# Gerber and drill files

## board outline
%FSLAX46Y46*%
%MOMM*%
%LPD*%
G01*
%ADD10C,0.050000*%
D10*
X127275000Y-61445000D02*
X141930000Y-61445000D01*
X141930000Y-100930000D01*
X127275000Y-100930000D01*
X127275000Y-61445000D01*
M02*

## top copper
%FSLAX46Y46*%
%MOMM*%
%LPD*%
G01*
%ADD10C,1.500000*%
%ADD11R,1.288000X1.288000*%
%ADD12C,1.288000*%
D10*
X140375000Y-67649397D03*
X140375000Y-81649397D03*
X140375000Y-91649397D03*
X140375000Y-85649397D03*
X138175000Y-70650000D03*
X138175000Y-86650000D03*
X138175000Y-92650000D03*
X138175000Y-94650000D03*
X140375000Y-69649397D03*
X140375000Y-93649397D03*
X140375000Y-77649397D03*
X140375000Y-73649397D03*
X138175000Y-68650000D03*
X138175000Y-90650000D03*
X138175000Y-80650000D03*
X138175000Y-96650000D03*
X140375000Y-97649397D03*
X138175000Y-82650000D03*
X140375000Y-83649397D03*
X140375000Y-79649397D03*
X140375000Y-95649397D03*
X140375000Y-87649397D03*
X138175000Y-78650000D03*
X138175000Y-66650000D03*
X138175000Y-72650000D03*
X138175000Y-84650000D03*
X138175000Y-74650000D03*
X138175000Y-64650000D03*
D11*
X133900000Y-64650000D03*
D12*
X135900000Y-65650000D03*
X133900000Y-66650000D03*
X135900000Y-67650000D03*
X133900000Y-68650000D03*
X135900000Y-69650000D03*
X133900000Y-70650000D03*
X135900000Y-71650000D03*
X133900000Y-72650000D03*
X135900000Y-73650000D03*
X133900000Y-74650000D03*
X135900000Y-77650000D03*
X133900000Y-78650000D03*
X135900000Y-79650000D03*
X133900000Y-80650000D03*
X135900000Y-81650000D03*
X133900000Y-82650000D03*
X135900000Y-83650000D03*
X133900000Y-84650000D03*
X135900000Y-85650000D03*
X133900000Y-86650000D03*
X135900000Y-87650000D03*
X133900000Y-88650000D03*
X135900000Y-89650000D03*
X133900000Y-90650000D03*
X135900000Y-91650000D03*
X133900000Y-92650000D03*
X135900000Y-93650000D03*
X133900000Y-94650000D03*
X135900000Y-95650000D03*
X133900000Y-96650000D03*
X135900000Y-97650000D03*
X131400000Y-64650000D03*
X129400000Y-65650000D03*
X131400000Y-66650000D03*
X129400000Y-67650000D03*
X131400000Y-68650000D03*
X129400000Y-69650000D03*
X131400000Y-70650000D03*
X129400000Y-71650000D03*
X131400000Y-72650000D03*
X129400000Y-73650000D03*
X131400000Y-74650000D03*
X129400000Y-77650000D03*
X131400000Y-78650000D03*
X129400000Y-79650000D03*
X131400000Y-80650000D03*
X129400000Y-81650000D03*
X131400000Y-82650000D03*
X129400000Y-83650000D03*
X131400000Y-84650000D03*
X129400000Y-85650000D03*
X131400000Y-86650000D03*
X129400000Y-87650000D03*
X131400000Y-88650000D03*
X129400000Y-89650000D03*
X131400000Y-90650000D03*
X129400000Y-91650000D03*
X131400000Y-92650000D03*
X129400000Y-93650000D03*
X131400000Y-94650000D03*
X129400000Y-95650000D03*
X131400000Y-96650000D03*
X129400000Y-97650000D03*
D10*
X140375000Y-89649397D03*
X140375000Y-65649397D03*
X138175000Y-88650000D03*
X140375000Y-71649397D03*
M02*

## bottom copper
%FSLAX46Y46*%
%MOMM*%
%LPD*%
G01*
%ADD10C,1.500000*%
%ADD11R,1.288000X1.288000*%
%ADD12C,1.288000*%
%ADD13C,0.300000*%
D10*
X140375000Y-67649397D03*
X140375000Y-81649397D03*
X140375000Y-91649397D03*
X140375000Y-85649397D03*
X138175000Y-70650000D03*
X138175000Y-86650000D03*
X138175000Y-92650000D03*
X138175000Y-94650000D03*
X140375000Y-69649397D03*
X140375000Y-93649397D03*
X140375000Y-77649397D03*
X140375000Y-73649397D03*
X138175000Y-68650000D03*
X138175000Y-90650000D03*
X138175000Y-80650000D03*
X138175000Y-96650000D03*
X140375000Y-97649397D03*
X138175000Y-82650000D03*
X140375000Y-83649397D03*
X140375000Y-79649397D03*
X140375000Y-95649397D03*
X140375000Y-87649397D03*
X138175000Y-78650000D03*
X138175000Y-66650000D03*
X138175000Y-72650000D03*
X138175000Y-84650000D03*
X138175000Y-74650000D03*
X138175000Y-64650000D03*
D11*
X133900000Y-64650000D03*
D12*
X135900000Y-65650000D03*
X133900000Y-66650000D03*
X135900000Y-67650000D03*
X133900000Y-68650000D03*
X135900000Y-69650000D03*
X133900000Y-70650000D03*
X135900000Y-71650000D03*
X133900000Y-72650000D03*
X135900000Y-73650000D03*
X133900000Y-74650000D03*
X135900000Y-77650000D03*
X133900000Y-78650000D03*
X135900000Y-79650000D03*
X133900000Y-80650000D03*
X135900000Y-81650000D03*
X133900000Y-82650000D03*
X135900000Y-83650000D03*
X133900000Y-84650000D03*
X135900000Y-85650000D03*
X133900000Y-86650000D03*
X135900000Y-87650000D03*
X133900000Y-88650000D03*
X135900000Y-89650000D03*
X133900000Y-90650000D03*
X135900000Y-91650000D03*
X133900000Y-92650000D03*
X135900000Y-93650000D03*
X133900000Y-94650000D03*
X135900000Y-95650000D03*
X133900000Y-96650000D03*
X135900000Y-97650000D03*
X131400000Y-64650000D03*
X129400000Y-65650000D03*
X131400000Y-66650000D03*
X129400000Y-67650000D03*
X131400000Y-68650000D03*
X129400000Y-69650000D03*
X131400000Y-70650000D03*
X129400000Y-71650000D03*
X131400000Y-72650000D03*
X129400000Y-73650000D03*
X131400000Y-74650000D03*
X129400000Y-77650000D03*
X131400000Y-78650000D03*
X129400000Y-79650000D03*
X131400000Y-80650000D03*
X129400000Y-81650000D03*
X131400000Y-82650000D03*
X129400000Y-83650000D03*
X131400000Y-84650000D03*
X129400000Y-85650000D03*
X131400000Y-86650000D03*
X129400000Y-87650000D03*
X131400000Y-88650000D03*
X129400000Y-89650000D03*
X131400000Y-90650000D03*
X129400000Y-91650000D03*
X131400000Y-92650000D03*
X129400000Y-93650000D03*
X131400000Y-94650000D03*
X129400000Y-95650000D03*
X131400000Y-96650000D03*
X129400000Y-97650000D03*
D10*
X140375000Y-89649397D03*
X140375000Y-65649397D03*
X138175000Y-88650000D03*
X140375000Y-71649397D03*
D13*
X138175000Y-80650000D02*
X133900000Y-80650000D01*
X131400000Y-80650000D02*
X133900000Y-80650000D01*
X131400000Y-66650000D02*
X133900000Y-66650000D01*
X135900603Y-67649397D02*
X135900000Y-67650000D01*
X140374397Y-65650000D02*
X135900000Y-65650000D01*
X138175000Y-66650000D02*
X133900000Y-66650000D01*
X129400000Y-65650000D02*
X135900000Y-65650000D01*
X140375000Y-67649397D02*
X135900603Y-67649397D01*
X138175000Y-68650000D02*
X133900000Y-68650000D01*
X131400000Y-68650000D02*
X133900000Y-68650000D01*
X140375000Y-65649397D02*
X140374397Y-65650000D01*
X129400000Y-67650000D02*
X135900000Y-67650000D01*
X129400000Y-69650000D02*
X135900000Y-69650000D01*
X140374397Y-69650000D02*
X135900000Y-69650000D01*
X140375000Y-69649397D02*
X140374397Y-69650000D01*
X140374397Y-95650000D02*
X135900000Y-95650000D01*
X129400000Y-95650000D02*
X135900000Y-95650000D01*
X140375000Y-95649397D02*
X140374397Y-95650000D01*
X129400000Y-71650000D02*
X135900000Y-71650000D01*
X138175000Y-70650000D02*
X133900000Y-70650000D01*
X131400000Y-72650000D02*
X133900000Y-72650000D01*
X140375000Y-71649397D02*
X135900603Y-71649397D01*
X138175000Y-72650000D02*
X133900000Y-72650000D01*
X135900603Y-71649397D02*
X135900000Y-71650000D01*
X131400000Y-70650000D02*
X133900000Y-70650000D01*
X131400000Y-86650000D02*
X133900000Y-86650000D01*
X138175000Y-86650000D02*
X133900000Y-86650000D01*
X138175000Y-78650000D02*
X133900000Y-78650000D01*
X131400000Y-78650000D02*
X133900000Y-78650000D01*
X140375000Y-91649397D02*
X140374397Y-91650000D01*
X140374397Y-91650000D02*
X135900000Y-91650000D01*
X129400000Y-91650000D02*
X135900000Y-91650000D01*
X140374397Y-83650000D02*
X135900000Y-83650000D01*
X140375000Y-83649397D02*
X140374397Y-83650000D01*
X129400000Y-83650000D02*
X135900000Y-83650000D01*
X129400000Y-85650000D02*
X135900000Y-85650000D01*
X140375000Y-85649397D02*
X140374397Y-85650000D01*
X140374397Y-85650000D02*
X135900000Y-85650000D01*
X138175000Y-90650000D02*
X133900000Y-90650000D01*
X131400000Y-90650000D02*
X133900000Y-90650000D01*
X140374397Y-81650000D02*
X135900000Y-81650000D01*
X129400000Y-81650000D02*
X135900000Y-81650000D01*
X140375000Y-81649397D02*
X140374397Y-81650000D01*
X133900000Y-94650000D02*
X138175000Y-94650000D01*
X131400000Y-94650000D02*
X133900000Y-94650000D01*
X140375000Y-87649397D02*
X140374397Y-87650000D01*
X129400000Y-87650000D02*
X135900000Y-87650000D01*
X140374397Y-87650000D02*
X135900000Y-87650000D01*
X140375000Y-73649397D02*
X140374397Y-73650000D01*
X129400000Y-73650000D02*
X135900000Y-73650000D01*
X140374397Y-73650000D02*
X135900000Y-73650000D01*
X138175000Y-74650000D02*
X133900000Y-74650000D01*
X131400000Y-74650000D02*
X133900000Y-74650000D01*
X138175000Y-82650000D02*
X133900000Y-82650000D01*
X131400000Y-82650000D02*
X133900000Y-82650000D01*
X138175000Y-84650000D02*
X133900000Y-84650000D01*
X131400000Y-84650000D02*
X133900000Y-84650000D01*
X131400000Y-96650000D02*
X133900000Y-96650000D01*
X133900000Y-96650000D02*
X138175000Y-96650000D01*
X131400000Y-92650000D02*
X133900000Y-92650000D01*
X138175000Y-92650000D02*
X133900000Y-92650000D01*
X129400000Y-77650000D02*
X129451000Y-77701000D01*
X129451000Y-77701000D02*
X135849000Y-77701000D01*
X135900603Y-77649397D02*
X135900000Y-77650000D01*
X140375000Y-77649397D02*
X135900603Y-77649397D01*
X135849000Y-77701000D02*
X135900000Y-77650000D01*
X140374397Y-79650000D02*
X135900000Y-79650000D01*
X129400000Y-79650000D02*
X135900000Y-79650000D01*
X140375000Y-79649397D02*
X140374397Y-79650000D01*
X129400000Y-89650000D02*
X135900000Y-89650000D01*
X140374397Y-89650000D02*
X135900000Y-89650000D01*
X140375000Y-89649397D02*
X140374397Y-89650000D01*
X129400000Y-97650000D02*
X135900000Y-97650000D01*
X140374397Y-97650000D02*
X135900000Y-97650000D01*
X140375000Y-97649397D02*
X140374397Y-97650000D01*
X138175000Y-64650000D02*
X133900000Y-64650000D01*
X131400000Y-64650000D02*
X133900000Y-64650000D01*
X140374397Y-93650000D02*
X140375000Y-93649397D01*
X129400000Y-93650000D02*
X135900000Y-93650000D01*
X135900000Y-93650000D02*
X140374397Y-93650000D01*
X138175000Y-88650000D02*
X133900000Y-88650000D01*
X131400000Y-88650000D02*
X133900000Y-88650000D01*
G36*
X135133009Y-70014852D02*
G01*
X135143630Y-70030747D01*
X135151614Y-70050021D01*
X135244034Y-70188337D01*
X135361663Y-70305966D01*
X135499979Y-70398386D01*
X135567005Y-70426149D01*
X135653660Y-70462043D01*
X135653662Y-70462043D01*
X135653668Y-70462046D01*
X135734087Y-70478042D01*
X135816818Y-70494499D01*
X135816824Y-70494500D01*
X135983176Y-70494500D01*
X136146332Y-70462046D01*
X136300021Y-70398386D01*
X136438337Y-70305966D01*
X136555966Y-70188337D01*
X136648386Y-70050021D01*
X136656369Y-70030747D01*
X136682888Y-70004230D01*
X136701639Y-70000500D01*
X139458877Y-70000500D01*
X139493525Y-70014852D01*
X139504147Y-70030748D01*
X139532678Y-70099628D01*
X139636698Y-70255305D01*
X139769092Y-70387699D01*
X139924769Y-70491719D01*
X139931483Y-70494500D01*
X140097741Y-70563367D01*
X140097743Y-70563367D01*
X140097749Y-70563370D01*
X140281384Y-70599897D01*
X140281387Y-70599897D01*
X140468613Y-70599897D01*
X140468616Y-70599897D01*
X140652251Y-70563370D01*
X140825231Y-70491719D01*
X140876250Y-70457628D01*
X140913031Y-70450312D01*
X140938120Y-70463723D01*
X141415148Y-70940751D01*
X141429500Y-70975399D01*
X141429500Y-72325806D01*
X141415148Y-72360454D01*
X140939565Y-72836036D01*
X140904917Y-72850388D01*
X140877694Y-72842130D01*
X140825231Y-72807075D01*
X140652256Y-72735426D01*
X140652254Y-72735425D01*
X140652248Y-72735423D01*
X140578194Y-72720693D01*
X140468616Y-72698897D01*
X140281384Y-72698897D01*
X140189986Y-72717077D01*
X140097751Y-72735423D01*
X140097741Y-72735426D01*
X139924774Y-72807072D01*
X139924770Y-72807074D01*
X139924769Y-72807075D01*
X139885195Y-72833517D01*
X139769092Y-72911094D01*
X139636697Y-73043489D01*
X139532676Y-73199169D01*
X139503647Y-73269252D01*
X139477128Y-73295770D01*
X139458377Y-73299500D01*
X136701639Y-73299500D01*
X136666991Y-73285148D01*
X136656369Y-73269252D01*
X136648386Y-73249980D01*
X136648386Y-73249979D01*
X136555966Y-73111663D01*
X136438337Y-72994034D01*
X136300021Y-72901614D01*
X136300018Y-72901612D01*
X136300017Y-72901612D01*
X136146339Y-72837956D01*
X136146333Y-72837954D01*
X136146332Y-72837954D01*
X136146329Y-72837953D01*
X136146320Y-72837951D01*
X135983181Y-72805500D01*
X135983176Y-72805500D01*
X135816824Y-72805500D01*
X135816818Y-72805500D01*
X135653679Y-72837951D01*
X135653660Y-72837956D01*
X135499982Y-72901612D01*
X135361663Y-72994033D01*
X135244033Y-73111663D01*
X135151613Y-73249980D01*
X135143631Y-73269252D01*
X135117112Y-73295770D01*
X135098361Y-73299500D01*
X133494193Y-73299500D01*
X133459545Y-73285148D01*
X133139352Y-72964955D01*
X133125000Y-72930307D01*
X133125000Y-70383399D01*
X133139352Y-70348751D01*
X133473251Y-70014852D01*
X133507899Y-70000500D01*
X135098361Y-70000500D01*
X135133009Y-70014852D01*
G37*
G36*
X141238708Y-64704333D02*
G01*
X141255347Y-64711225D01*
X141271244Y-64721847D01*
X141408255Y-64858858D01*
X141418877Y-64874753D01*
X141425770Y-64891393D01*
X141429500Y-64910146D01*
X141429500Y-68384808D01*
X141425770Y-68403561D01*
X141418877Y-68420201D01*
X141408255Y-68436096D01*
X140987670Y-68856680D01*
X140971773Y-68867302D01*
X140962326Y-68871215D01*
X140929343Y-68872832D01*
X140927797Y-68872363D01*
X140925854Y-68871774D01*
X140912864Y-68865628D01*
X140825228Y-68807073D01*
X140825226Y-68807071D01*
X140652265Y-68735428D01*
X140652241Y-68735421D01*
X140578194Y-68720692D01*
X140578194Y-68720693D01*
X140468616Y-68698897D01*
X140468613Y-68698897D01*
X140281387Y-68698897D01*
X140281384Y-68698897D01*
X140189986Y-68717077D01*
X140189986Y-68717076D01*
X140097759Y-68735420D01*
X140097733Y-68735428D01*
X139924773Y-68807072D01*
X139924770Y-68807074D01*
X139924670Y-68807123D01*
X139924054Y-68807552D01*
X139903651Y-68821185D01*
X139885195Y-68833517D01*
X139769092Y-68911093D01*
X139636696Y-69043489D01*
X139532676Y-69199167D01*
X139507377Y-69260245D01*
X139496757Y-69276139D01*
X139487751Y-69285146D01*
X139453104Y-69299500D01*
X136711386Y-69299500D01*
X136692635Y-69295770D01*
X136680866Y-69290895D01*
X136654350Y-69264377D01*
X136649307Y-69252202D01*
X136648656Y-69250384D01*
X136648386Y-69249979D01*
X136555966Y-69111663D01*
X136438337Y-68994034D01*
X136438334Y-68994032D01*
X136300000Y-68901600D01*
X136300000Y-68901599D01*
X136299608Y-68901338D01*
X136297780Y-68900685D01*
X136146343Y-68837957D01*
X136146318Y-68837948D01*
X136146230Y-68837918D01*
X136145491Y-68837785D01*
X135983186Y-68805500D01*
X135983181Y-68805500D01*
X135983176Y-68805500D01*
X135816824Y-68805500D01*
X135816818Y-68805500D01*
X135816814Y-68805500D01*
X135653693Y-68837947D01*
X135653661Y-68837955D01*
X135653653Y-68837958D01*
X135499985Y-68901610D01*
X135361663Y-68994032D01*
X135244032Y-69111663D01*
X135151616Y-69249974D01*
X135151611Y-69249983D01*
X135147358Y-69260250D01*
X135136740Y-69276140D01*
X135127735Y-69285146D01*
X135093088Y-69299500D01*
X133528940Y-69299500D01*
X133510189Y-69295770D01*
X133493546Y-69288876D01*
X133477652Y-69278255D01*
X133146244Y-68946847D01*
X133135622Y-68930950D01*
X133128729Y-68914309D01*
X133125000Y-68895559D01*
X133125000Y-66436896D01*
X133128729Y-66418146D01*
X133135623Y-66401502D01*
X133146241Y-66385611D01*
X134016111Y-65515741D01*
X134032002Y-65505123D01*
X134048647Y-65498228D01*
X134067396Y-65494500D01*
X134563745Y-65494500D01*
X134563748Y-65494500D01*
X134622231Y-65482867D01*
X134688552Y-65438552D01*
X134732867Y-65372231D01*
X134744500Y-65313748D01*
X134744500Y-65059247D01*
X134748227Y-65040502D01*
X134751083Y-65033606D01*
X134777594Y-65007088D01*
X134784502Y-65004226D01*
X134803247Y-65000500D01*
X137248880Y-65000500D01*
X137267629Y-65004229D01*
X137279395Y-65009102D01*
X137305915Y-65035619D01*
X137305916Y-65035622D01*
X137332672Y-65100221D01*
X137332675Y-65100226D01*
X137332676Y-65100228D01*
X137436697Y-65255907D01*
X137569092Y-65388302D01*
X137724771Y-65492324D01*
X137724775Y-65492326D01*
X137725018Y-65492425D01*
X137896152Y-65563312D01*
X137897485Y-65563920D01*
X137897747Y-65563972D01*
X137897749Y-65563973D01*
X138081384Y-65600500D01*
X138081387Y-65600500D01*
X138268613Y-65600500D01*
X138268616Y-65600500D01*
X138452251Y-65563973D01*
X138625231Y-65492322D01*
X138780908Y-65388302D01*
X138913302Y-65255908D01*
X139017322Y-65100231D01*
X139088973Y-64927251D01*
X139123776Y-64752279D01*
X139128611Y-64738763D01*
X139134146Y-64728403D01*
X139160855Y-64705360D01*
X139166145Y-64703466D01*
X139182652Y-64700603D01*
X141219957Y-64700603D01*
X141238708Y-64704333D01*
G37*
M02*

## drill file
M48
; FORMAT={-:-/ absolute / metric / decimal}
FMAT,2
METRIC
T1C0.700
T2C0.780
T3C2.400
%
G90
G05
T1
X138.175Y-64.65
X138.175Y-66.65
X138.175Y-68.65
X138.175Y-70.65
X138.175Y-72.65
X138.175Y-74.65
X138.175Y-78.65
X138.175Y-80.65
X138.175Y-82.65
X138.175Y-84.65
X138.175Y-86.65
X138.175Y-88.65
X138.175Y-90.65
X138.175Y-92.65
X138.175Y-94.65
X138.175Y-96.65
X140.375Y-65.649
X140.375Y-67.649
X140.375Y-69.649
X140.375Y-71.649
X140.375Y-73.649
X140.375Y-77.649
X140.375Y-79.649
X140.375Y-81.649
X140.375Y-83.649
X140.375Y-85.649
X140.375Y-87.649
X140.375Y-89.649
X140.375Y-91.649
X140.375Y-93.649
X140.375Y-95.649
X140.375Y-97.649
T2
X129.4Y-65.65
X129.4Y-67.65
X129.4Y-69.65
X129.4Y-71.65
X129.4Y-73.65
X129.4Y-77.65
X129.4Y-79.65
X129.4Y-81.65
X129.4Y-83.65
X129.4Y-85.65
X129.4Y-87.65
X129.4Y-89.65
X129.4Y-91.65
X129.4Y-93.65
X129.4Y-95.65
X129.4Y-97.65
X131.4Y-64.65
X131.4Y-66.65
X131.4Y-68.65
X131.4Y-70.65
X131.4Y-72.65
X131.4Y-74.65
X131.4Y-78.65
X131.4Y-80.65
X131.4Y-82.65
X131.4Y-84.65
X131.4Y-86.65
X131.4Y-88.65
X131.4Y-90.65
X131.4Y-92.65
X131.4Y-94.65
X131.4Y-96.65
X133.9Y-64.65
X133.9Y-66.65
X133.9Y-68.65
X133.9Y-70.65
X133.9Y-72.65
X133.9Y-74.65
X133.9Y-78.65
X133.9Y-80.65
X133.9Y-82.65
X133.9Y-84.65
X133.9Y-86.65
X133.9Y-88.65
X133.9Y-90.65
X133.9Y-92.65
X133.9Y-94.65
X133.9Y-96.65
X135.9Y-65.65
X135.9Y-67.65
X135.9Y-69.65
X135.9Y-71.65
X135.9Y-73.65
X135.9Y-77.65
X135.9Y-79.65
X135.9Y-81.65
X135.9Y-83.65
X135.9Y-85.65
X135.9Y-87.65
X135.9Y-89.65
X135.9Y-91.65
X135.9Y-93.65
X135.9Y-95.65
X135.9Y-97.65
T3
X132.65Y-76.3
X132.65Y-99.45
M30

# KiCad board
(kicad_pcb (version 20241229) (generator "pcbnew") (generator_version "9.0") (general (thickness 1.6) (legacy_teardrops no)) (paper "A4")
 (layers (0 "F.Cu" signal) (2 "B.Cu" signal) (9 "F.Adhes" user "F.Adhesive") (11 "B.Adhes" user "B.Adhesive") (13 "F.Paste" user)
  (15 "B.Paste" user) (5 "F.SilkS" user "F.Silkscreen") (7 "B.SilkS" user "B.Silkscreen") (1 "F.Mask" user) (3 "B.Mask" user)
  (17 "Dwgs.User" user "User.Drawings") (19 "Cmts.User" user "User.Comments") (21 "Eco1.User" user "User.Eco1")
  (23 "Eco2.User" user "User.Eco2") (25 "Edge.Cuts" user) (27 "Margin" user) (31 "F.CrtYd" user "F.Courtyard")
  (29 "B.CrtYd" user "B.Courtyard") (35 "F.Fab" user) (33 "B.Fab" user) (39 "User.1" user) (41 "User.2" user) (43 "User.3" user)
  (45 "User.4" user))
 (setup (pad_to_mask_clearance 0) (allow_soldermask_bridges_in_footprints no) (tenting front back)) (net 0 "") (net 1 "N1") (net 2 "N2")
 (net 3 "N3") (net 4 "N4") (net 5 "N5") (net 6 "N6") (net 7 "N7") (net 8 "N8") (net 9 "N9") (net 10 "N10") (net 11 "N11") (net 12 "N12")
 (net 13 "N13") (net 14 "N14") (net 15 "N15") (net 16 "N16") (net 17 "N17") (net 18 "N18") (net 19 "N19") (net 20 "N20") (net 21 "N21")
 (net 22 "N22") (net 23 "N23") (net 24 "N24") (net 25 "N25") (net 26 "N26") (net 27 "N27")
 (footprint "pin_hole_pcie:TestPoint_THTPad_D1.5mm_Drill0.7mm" (layer "F.Cu") (at 140.375 67.649397 180)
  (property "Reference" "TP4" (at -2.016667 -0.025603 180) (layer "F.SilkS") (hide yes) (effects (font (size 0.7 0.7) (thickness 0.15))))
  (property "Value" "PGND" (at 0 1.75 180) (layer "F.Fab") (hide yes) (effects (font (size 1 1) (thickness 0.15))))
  (pad "1" thru_hole circle (at 0 0 180) (size 1.5 1.5) (drill 0.7) (layers "*.Cu" "*.Mask") (remove_unused_layers no) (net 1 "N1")))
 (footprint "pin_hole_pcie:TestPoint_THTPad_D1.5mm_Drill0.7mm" (layer "F.Cu") (at 140.375 81.649397 180)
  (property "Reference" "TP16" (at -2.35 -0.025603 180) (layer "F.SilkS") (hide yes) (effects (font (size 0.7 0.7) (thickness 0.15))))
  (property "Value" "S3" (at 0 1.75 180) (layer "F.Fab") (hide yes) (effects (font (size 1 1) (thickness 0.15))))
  (pad "1" thru_hole circle (at 0 0 180) (size 1.5 1.5) (drill 0.7) (layers "*.Cu" "*.Mask") (remove_unused_layers no) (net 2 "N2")))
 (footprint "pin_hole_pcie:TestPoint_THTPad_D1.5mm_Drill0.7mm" (layer "F.Cu") (at 140.375 91.649397 180)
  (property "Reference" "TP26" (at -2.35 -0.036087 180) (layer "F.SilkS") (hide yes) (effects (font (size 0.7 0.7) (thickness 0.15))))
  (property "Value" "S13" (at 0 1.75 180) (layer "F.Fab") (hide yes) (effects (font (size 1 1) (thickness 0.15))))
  (pad "1" thru_hole circle (at 0 0 180) (size 1.5 1.5) (drill 0.7) (layers "*.Cu" "*.Mask") (remove_unused_layers no) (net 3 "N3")))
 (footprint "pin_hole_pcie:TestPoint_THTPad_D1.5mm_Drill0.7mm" (layer "F.Cu") (at 140.375 85.649397 180)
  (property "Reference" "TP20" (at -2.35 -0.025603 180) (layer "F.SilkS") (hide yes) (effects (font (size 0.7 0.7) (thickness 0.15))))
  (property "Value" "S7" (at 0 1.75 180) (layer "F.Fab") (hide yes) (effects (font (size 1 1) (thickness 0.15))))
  (pad "1" thru_hole circle (at 0 0 180) (size 1.5 1.5) (drill 0.7) (layers "*.Cu" "*.Mask") (remove_unused_layers no) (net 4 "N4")))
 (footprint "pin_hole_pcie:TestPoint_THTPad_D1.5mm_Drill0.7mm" (layer "F.Cu") (at 138.175 70.65 180)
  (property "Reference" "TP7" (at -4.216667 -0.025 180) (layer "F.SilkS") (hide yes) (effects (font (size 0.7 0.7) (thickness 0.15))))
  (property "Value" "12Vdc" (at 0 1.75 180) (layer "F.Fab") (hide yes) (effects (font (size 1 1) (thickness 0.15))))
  (pad "1" thru_hole circle (at 0 0 180) (size 1.5 1.5) (drill 0.7) (layers "*.Cu" "*.Mask") (remove_unused_layers no) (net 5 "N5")))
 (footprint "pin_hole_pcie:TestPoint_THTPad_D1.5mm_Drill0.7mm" (layer "F.Cu") (at 138.175 86.65 180)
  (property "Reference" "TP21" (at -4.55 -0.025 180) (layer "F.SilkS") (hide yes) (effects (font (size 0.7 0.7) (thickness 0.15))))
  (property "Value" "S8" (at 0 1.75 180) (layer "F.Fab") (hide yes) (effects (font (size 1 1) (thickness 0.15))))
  (pad "1" thru_hole circle (at 0 0 180) (size 1.5 1.5) (drill 0.7) (layers "*.Cu" "*.Mask") (remove_unused_layers no) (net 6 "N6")))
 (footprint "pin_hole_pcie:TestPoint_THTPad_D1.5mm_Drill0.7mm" (layer "F.Cu") (at 138.175 92.65 180)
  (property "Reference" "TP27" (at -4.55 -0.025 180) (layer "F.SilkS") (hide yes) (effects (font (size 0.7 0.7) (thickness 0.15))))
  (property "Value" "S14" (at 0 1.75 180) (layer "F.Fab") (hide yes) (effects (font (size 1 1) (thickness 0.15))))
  (pad "1" thru_hole circle (at 0 0 180) (size 1.5 1.5) (drill 0.7) (layers "*.Cu" "*.Mask") (remove_unused_layers no) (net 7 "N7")))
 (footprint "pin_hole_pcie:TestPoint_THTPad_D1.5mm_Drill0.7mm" (layer "F.Cu") (at 138.175 94.65 180)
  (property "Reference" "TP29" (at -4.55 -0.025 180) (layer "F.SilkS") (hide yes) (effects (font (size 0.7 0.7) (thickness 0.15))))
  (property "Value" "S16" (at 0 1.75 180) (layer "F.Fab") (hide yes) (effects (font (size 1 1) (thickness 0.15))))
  (pad "1" thru_hole circle (at 0 0 180) (size 1.5 1.5) (drill 0.7) (layers "*.Cu" "*.Mask") (remove_unused_layers no) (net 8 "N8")))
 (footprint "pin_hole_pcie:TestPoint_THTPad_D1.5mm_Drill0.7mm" (layer "F.Cu") (at 140.375 69.649397 180)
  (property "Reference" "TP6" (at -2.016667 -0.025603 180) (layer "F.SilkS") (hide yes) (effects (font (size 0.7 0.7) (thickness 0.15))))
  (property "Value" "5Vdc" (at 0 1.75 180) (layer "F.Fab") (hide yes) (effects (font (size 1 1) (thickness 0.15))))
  (pad "1" thru_hole circle (at 0 0 180) (size 1.5 1.5) (drill 0.7) (layers "*.Cu" "*.Mask") (remove_unused_layers no) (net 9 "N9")))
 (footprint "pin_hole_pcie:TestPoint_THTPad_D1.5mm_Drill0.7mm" (layer "F.Cu") (at 140.375 93.649397 180)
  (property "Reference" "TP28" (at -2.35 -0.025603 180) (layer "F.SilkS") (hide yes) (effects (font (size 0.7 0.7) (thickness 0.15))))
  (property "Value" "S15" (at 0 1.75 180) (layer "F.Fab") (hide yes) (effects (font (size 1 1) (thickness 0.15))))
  (pad "1" thru_hole circle (at 0 0 180) (size 1.5 1.5) (drill 0.7) (layers "*.Cu" "*.Mask") (remove_unused_layers no) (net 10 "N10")))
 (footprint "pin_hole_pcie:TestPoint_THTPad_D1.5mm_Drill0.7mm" (layer "F.Cu") (at 140.375 77.649397 180)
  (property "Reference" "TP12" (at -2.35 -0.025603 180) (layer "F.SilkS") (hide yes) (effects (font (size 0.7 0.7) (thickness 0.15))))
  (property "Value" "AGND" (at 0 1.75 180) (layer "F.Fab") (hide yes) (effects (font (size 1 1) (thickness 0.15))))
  (pad "1" thru_hole circle (at 0 0 180) (size 1.5 1.5) (drill 0.7) (layers "*.Cu" "*.Mask") (remove_unused_layers no) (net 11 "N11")))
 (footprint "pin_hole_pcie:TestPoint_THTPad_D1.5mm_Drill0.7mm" (layer "F.Cu") (at 140.375 73.649397 180)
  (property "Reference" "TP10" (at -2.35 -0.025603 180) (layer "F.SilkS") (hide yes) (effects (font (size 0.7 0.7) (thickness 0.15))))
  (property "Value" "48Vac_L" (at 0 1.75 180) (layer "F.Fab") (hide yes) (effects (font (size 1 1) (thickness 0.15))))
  (pad "1" thru_hole circle (at 0 0 180) (size 1.5 1.5) (drill 0.7) (layers "*.Cu" "*.Mask") (remove_unused_layers no) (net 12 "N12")))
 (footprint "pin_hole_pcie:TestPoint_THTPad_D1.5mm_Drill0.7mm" (layer "F.Cu") (at 138.175 68.65 180)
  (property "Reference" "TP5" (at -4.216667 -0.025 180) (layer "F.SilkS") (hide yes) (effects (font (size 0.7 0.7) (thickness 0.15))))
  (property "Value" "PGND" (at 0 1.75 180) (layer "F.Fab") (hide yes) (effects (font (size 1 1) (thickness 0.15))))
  (pad "1" thru_hole circle (at 0 0 180) (size 1.5 1.5) (drill 0.7) (layers "*.Cu" "*.Mask") (remove_unused_layers no) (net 1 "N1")))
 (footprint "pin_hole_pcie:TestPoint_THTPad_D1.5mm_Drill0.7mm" (layer "F.Cu") (at 138.175 90.65 180)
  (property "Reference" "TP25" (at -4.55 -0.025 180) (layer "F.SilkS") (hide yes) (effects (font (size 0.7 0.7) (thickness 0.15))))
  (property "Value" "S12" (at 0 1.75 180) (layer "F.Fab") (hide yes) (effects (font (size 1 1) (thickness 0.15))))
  (pad "1" thru_hole circle (at 0 0 180) (size 1.5 1.5) (drill 0.7) (layers "*.Cu" "*.Mask") (remove_unused_layers no) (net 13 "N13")))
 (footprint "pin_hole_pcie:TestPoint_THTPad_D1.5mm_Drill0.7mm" (layer "F.Cu") (at 138.175 80.65 180)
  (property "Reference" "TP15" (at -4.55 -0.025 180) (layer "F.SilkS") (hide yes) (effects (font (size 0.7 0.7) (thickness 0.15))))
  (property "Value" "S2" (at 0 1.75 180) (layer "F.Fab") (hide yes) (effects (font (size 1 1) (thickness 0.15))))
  (pad "1" thru_hole circle (at 0 0 180) (size 1.5 1.5) (drill 0.7) (layers "*.Cu" "*.Mask") (remove_unused_layers no) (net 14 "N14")))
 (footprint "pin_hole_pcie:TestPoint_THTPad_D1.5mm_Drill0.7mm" (layer "F.Cu") (at 138.175 96.65 180)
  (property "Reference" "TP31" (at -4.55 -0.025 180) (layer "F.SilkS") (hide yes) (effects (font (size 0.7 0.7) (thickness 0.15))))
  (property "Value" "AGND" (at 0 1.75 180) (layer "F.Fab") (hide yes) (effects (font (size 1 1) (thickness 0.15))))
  (pad "1" thru_hole circle (at 0 0 180) (size 1.5 1.5) (drill 0.7) (layers "*.Cu" "*.Mask") (remove_unused_layers no) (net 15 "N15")))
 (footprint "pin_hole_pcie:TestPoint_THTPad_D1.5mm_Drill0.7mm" (layer "F.Cu") (at 140.375 97.649397 180)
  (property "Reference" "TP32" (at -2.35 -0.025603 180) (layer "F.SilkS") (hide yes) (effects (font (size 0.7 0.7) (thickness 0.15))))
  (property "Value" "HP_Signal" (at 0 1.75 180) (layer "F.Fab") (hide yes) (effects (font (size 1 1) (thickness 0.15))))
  (pad "1" thru_hole circle (at 0 0 180) (size 1.5 1.5) (drill 0.7) (layers "*.Cu" "*.Mask") (remove_unused_layers no) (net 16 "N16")))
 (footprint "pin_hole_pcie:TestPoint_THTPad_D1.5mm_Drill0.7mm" (layer "F.Cu") (at 138.175 82.65 180)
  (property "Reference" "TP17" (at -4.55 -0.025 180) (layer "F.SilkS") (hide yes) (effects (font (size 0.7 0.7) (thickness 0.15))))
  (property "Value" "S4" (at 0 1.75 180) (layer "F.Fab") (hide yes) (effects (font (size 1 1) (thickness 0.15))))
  (pad "1" thru_hole circle (at 0 0 180) (size 1.5 1.5) (drill 0.7) (layers "*.Cu" "*.Mask") (remove_unused_layers no) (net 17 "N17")))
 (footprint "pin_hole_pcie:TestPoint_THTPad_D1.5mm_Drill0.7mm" (layer "F.Cu") (at 140.375 83.649397 180)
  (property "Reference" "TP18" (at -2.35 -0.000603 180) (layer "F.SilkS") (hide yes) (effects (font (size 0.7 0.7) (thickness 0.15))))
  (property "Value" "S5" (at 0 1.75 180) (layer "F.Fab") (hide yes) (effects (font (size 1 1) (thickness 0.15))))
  (pad "1" thru_hole circle (at 0 0 180) (size 1.5 1.5) (drill 0.7) (layers "*.Cu" "*.Mask") (remove_unused_layers no) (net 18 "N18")))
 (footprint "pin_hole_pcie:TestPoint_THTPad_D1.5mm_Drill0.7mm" (layer "F.Cu") (at 140.375 79.649397 180)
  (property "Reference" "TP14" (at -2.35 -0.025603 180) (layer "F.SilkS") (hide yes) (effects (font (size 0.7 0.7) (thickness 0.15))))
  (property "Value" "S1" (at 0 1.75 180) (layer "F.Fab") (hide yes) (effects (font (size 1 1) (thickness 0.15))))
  (pad "1" thru_hole circle (at 0 0 180) (size 1.5 1.5) (drill 0.7) (layers "*.Cu" "*.Mask") (remove_unused_layers no) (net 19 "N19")))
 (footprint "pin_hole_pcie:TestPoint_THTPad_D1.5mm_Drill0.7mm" (layer "F.Cu") (at 140.375 95.649397 180)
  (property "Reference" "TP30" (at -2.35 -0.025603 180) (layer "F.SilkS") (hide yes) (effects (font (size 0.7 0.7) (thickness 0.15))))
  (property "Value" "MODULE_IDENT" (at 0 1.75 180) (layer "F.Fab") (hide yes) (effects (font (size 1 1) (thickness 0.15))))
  (pad "1" thru_hole circle (at 0 0 180) (size 1.5 1.5) (drill 0.7) (layers "*.Cu" "*.Mask") (remove_unused_layers no) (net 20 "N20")))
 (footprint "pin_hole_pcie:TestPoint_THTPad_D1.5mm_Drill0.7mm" (layer "F.Cu") (at 140.375 87.649397 180)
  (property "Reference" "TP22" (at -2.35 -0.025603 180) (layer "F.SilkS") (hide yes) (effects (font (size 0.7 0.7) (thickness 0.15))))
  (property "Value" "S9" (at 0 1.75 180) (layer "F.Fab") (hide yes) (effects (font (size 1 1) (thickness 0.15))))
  (pad "1" thru_hole circle (at 0 0 180) (size 1.5 1.5) (drill 0.7) (layers "*.Cu" "*.Mask") (remove_unused_layers no) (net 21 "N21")))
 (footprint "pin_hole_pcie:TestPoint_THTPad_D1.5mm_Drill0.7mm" (layer "F.Cu") (at 138.175 78.65 180)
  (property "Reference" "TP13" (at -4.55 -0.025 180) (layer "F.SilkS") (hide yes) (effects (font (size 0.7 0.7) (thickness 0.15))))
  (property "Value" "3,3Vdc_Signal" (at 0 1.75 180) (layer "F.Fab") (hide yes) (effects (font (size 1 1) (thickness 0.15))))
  (pad "1" thru_hole circle (at 0 0 180) (size 1.5 1.5) (drill 0.7) (layers "*.Cu" "*.Mask") (remove_unused_layers no) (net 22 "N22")))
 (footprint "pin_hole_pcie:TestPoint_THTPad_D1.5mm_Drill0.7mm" (layer "F.Cu") (at 138.175 66.65 180)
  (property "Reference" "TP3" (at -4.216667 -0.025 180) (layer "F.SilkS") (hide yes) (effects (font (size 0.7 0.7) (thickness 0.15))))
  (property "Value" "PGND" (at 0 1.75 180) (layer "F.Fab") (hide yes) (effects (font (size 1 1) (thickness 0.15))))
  (pad "1" thru_hole circle (at 0 0 180) (size 1.5 1.5) (drill 0.7) (layers "*.Cu" "*.Mask") (remove_unused_layers no) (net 1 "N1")))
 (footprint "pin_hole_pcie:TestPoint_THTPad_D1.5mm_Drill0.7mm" (layer "F.Cu") (at 138.175 72.65 180)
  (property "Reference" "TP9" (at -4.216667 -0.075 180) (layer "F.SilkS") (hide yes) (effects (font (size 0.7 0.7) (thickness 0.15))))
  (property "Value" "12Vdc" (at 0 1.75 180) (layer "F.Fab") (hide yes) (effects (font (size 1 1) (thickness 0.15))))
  (pad "1" thru_hole circle (at 0 0 180) (size 1.5 1.5) (drill 0.7) (layers "*.Cu" "*.Mask") (remove_unused_layers no) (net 5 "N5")))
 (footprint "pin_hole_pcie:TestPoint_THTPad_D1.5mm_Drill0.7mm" (layer "F.Cu") (at 138.175 84.65 180)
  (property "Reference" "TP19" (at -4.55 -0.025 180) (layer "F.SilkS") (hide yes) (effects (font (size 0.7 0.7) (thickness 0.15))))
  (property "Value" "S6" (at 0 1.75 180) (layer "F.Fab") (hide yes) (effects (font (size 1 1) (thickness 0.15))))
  (pad "1" thru_hole circle (at 0 0 180) (size 1.5 1.5) (drill 0.7) (layers "*.Cu" "*.Mask") (remove_unused_layers no) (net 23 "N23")))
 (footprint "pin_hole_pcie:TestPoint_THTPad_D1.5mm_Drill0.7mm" (layer "F.Cu") (at 138.175 74.65 180)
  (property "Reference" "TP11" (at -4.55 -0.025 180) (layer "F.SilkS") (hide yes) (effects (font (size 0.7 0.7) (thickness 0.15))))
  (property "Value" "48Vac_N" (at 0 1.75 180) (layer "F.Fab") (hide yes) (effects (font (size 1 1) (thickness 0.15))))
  (pad "1" thru_hole circle (at 0 0 180) (size 1.5 1.5) (drill 0.7) (layers "*.Cu" "*.Mask") (remove_unused_layers no) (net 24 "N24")))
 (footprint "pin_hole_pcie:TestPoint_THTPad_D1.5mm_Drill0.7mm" (layer "F.Cu") (at 138.175 64.65 180)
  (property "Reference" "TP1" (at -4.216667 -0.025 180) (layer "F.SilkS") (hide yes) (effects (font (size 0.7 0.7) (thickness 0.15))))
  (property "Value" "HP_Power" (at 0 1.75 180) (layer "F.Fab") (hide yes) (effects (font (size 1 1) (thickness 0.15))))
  (pad "1" thru_hole circle (at 0 0 180) (size 1.5 1.5) (drill 0.7) (layers "*.Cu" "*.Mask") (remove_unused_layers no) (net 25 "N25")))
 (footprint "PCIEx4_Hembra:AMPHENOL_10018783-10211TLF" (layer "F.Cu") (at 132.65 76.3 -90)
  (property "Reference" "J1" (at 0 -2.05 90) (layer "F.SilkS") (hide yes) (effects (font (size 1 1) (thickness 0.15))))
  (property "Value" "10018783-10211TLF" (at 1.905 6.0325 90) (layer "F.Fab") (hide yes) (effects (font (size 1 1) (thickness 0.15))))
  (pad "" np_thru_hole circle (at 0 0 270) (size 2.4 2.4) (drill 2.4) (layers "*.Cu" "*.Mask"))
  (pad "" np_thru_hole circle (at 23.15 0 270) (size 2.4 2.4) (drill 2.4) (layers "*.Cu" "*.Mask"))
  (pad "A1" thru_hole rect (at -11.65 -1.25 270) (size 1.288 1.288) (drill 0.78) (layers "*.Cu" "*.Mask") (remove_unused_layers no)
   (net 25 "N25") (solder_mask_margin 0.102))
  (pad "A2" thru_hole circle (at -10.65 -3.25 270) (size 1.288 1.288) (drill 0.78) (layers "*.Cu" "*.Mask") (remove_unused_layers no)
   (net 1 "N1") (solder_mask_margin 0.102))
  (pad "A3" thru_hole circle (at -9.65 -1.25 270) (size 1.288 1.288) (drill 0.78) (layers "*.Cu" "*.Mask") (remove_unused_layers no)
   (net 1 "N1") (solder_mask_margin 0.102))
  (pad "A4" thru_hole circle (at -8.65 -3.25 270) (size 1.288 1.288) (drill 0.78) (layers "*.Cu" "*.Mask") (remove_unused_layers no)
   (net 1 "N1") (solder_mask_margin 0.102))
  (pad "A5" thru_hole circle (at -7.65 -1.25 270) (size 1.288 1.288) (drill 0.78) (layers "*.Cu" "*.Mask") (remove_unused_layers no)
   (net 1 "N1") (solder_mask_margin 0.102))
  (pad "A6" thru_hole circle (at -6.65 -3.25 270) (size 1.288 1.288) (drill 0.78) (layers "*.Cu" "*.Mask") (remove_unused_layers no)
   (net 9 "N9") (solder_mask_margin 0.102))
  (pad "A7" thru_hole circle (at -5.65 -1.25 270) (size 1.288 1.288) (drill 0.78) (layers "*.Cu" "*.Mask") (remove_unused_layers no)
   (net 5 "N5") (solder_mask_margin 0.102))
  (pad "A8" thru_hole circle (at -4.65 -3.25 270) (size 1.288 1.288) (drill 0.78) (layers "*.Cu" "*.Mask") (remove_unused_layers no)
   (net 5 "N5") (solder_mask_margin 0.102))
  (pad "A9" thru_hole circle (at -3.65 -1.25 270) (size 1.288 1.288) (drill 0.78) (layers "*.Cu" "*.Mask") (remove_unused_layers no)
   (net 5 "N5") (solder_mask_margin 0.102))
  (pad "A10" thru_hole circle (at -2.65 -3.25 270) (size 1.288 1.288) (drill 0.78) (layers "*.Cu" "*.Mask") (remove_unused_layers no)
   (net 12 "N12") (solder_mask_margin 0.102))
  (pad "A11" thru_hole circle (at -1.65 -1.25 270) (size 1.288 1.288) (drill 0.78) (layers "*.Cu" "*.Mask") (remove_unused_layers no)
   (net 24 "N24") (solder_mask_margin 0.102))
  (pad "A12" thru_hole circle (at 1.35 -3.25 270) (size 1.288 1.288) (drill 0.78) (layers "*.Cu" "*.Mask") (remove_unused_layers no)
   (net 11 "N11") (solder_mask_margin 0.102))
  (pad "A13" thru_hole circle (at 2.35 -1.25 270) (size 1.288 1.288) (drill 0.78) (layers "*.Cu" "*.Mask") (remove_unused_layers no)
   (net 22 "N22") (solder_mask_margin 0.102))
  (pad "A14" thru_hole circle (at 3.35 -3.25 270) (size 1.288 1.288) (drill 0.78) (layers "*.Cu" "*.Mask") (remove_unused_layers no)
   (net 19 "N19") (solder_mask_margin 0.102))
  (pad "A15" thru_hole circle (at 4.35 -1.25 270) (size 1.288 1.288) (drill 0.78) (layers "*.Cu" "*.Mask") (remove_unused_layers no)
   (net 14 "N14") (solder_mask_margin 0.102))
  (pad "A16" thru_hole circle (at 5.35 -3.25 270) (size 1.288 1.288) (drill 0.78) (layers "*.Cu" "*.Mask") (remove_unused_layers no)
   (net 2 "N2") (solder_mask_margin 0.102))
  (pad "A17" thru_hole circle (at 6.35 -1.25 270) (size 1.288 1.288) (drill 0.78) (layers "*.Cu" "*.Mask") (remove_unused_layers no)
   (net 17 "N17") (solder_mask_margin 0.102))
  (pad "A18" thru_hole circle (at 7.35 -3.25 270) (size 1.288 1.288) (drill 0.78) (layers "*.Cu" "*.Mask") (remove_unused_layers no)
   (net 18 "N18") (solder_mask_margin 0.102))
  (pad "A19" thru_hole circle (at 8.35 -1.25 270) (size 1.288 1.288) (drill 0.78) (layers "*.Cu" "*.Mask") (remove_unused_layers no)
   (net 23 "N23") (solder_mask_margin 0.102))
  (pad "A20" thru_hole circle (at 9.35 -3.25 270) (size 1.288 1.288) (drill 0.78) (layers "*.Cu" "*.Mask") (remove_unused_layers no)
   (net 4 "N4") (solder_mask_margin 0.102))
  (pad "A21" thru_hole circle (at 10.35 -1.25 270) (size 1.288 1.288) (drill 0.78) (layers "*.Cu" "*.Mask") (remove_unused_layers no)
   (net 6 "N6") (solder_mask_margin 0.102))
  (pad "A22" thru_hole circle (at 11.35 -3.25 270) (size 1.288 1.288) (drill 0.78) (layers "*.Cu" "*.Mask") (remove_unused_layers no)
   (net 21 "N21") (solder_mask_margin 0.102))
  (pad "A23" thru_hole circle (at 12.35 -1.25 270) (size 1.288 1.288) (drill 0.78) (layers "*.Cu" "*.Mask") (remove_unused_layers no)
   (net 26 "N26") (solder_mask_margin 0.102))
  (pad "A24" thru_hole circle (at 13.35 -3.25 270) (size 1.288 1.288) (drill 0.78) (layers "*.Cu" "*.Mask") (remove_unused_layers no)
   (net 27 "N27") (solder_mask_margin 0.102))
  (pad "A25" thru_hole circle (at 14.35 -1.25 270) (size 1.288 1.288) (drill 0.78) (layers "*.Cu" "*.Mask") (remove_unused_layers no)
   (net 13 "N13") (solder_mask_margin 0.102))
  (pad "A26" thru_hole circle (at 15.35 -3.25 270) (size 1.288 1.288) (drill 0.78) (layers "*.Cu" "*.Mask") (remove_unused_layers no)
   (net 3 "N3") (solder_mask_margin 0.102))
  (pad "A27" thru_hole circle (at 16.35 -1.25 270) (size 1.288 1.288) (drill 0.78) (layers "*.Cu" "*.Mask") (remove_unused_layers no)
   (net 7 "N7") (solder_mask_margin 0.102))
  (pad "A28" thru_hole circle (at 17.35 -3.25 270) (size 1.288 1.288) (drill 0.78) (layers "*.Cu" "*.Mask") (remove_unused_layers no)
   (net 10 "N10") (solder_mask_margin 0.102))
  (pad "A29" thru_hole circle (at 18.35 -1.25 270) (size 1.288 1.288) (drill 0.78) (layers "*.Cu" "*.Mask") (remove_unused_layers no)
   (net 8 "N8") (solder_mask_margin 0.102))
  (pad "A30" thru_hole circle (at 19.35 -3.25 270) (size 1.288 1.288) (drill 0.78) (layers "*.Cu" "*.Mask") (remove_unused_layers no)
   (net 20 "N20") (solder_mask_margin 0.102))
  (pad "A31" thru_hole circle (at 20.35 -1.25 270) (size 1.288 1.288) (drill 0.78) (layers "*.Cu" "*.Mask") (remove_unused_layers no)
   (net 15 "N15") (solder_mask_margin 0.102))
  (pad "A32" thru_hole circle (at 21.35 -3.25 270) (size 1.288 1.288) (drill 0.78) (layers "*.Cu" "*.Mask") (remove_unused_layers no)
   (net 16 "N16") (solder_mask_margin 0.102))
  (pad "B1" thru_hole circle (at -11.65 1.25 270) (size 1.288 1.288) (drill 0.78) (layers "*.Cu" "*.Mask") (remove_unused_layers no)
   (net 25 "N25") (solder_mask_margin 0.102))
  (pad "B2" thru_hole circle (at -10.65 3.25 270) (size 1.288 1.288) (drill 0.78) (layers "*.Cu" "*.Mask") (remove_unused_layers no)
   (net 1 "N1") (solder_mask_margin 0.102))
  (pad "B3" thru_hole circle (at -9.65 1.25 270) (size 1.288 1.288) (drill 0.78) (layers "*.Cu" "*.Mask") (remove_unused_layers no)
   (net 1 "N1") (solder_mask_margin 0.102))
  (pad "B4" thru_hole circle (at -8.65 3.25 270) (size 1.288 1.288) (drill 0.78) (layers "*.Cu" "*.Mask") (remove_unused_layers no)
   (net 1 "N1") (solder_mask_margin 0.102))
  (pad "B5" thru_hole circle (at -7.65 1.25 270) (size 1.288 1.288) (drill 0.78) (layers "*.Cu" "*.Mask") (remove_unused_layers no)
   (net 1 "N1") (solder_mask_margin 0.102))
  (pad "B6" thru_hole circle (at -6.65 3.25 270) (size 1.288 1.288) (drill 0.78) (layers "*.Cu" "*.Mask") (remove_unused_layers no)
   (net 9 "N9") (solder_mask_margin 0.102))
  (pad "B7" thru_hole circle (at -5.65 1.25 270) (size 1.288 1.288) (drill 0.78) (layers "*.Cu" "*.Mask") (remove_unused_layers no)
   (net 5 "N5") (solder_mask_margin 0.102))
  (pad "B8" thru_hole circle (at -4.65 3.25 270) (size 1.288 1.288) (drill 0.78) (layers "*.Cu" "*.Mask") (remove_unused_layers no)
   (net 5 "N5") (solder_mask_margin 0.102))
  (pad "B9" thru_hole circle (at -3.65 1.25 270) (size 1.288 1.288) (drill 0.78) (layers "*.Cu" "*.Mask") (remove_unused_layers no)
   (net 5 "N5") (solder_mask_margin 0.102))
  (pad "B10" thru_hole circle (at -2.65 3.25 270) (size 1.288 1.288) (drill 0.78) (layers "*.Cu" "*.Mask") (remove_unused_layers no)
   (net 12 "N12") (solder_mask_margin 0.102))
  (pad "B11" thru_hole circle (at -1.65 1.25 270) (size 1.288 1.288) (drill 0.78) (layers "*.Cu" "*.Mask") (remove_unused_layers no)
   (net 24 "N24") (solder_mask_margin 0.102))
  (pad "B12" thru_hole circle (at 1.35 3.25 270) (size 1.288 1.288) (drill 0.78) (layers "*.Cu" "*.Mask") (remove_unused_layers no)
   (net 11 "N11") (solder_mask_margin 0.102))
  (pad "B13" thru_hole circle (at 2.35 1.25 270) (size 1.288 1.288) (drill 0.78) (layers "*.Cu" "*.Mask") (remove_unused_layers no)
   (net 22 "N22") (solder_mask_margin 0.102))
  (pad "B14" thru_hole circle (at 3.35 3.25 270) (size 1.288 1.288) (drill 0.78) (layers "*.Cu" "*.Mask") (remove_unused_layers no)
   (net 19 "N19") (solder_mask_margin 0.102))
  (pad "B15" thru_hole circle (at 4.35 1.25 270) (size 1.288 1.288) (drill 0.78) (layers "*.Cu" "*.Mask") (remove_unused_layers no)
   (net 14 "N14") (solder_mask_margin 0.102))
  (pad "B16" thru_hole circle (at 5.35 3.25 270) (size 1.288 1.288) (drill 0.78) (layers "*.Cu" "*.Mask") (remove_unused_layers no)
   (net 2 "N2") (solder_mask_margin 0.102))
  (pad "B17" thru_hole circle (at 6.35 1.25 270) (size 1.288 1.288) (drill 0.78) (layers "*.Cu" "*.Mask") (remove_unused_layers no)
   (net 17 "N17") (solder_mask_margin 0.102))
  (pad "B18" thru_hole circle (at 7.35 3.25 270) (size 1.288 1.288) (drill 0.78) (layers "*.Cu" "*.Mask") (remove_unused_layers no)
   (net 18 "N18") (solder_mask_margin 0.102))
  (pad "B19" thru_hole circle (at 8.35 1.25 270) (size 1.288 1.288) (drill 0.78) (layers "*.Cu" "*.Mask") (remove_unused_layers no)
   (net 23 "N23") (solder_mask_margin 0.102))
  (pad "B20" thru_hole circle (at 9.35 3.25 270) (size 1.288 1.288) (drill 0.78) (layers "*.Cu" "*.Mask") (remove_unused_layers no)
   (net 4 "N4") (solder_mask_margin 0.102))
  (pad "B21" thru_hole circle (at 10.35 1.25 270) (size 1.288 1.288) (drill 0.78) (layers "*.Cu" "*.Mask") (remove_unused_layers no)
   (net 6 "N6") (solder_mask_margin 0.102))
  (pad "B22" thru_hole circle (at 11.35 3.25 270) (size 1.288 1.288) (drill 0.78) (layers "*.Cu" "*.Mask") (remove_unused_layers no)
   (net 21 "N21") (solder_mask_margin 0.102))
  (pad "B23" thru_hole circle (at 12.35 1.25 270) (size 1.288 1.288) (drill 0.78) (layers "*.Cu" "*.Mask") (remove_unused_layers no)
   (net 26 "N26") (solder_mask_margin 0.102))
  (pad "B24" thru_hole circle (at 13.35 3.25 270) (size 1.288 1.288) (drill 0.78) (layers "*.Cu" "*.Mask") (remove_unused_layers no)
   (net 27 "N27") (solder_mask_margin 0.102))
  (pad "B25" thru_hole circle (at 14.35 1.25 270) (size 1.288 1.288) (drill 0.78) (layers "*.Cu" "*.Mask") (remove_unused_layers no)
   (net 13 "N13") (solder_mask_margin 0.102))
  (pad "B26" thru_hole circle (at 15.35 3.25 270) (size 1.288 1.288) (drill 0.78) (layers "*.Cu" "*.Mask") (remove_unused_layers no)
   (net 3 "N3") (solder_mask_margin 0.102))
  (pad "B27" thru_hole circle (at 16.35 1.25 270) (size 1.288 1.288) (drill 0.78) (layers "*.Cu" "*.Mask") (remove_unused_layers no)
   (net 7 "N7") (solder_mask_margin 0.102))
  (pad "B28" thru_hole circle (at 17.35 3.25 270) (size 1.288 1.288) (drill 0.78) (layers "*.Cu" "*.Mask") (remove_unused_layers no)
   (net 10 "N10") (solder_mask_margin 0.102))
  (pad "B29" thru_hole circle (at 18.35 1.25 270) (size 1.288 1.288) (drill 0.78) (layers "*.Cu" "*.Mask") (remove_unused_layers no)
   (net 8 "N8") (solder_mask_margin 0.102))
  (pad "B30" thru_hole circle (at 19.35 3.25 270) (size 1.288 1.288) (drill 0.78) (layers "*.Cu" "*.Mask") (remove_unused_layers no)
   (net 20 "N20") (solder_mask_margin 0.102))
  (pad "B31" thru_hole circle (at 20.35 1.25 270) (size 1.288 1.288) (drill 0.78) (layers "*.Cu" "*.Mask") (remove_unused_layers no)
   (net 15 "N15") (solder_mask_margin 0.102))
  (pad "B32" thru_hole circle (at 21.35 3.25 270) (size 1.288 1.288) (drill 0.78) (layers "*.Cu" "*.Mask") (remove_unused_layers no)
   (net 16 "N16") (solder_mask_margin 0.102)))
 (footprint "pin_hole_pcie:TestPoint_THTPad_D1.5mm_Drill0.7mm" (layer "F.Cu") (at 140.375 89.649397 180)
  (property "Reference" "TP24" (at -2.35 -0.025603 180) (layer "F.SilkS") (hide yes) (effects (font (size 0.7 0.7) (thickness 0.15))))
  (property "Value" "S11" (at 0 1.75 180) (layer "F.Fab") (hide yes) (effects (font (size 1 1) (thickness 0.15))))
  (pad "1" thru_hole circle (at 0 0 180) (size 1.5 1.5) (drill 0.7) (layers "*.Cu" "*.Mask") (remove_unused_layers no) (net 27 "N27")))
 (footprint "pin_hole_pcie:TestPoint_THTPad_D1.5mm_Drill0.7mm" (layer "F.Cu") (at 140.375 65.649397 180)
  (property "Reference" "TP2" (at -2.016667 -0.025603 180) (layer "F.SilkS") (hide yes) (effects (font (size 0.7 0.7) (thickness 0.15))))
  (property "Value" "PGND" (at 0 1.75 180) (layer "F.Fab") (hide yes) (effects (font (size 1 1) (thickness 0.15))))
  (pad "1" thru_hole circle (at 0 0 180) (size 1.5 1.5) (drill 0.7) (layers "*.Cu" "*.Mask") (remove_unused_layers no) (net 1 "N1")))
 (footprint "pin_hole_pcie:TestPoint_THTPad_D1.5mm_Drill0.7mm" (layer "F.Cu") (at 138.175 88.65 180)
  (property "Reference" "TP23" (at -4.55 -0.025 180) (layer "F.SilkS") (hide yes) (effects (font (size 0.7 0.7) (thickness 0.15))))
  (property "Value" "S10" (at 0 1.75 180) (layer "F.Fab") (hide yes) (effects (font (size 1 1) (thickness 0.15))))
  (pad "1" thru_hole circle (at 0 0 180) (size 1.5 1.5) (drill 0.7) (layers "*.Cu" "*.Mask") (remove_unused_layers no) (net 26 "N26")))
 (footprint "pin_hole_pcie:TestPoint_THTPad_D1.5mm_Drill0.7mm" (layer "F.Cu") (at 140.375 71.649397 180)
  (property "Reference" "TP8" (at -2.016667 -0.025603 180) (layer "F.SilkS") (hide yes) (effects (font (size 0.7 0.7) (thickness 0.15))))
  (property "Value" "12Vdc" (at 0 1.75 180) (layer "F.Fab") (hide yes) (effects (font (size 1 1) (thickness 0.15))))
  (pad "1" thru_hole circle (at 0 0 180) (size 1.5 1.5) (drill 0.7) (layers "*.Cu" "*.Mask") (remove_unused_layers no) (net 5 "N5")))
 (gr_rect (start 127.275 61.445) (end 141.93 100.93) (stroke (width 0.05) (type default)) (fill no) (layer "Edge.Cuts"))
 (segment (start 138.175 80.65) (end 133.9 80.65) (width 0.3) (layer "B.Cu") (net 14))
 (segment (start 131.4 80.65) (end 133.9 80.65) (width 0.3) (layer "B.Cu") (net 14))
 (segment (start 131.4 66.65) (end 133.9 66.65) (width 0.3) (layer "B.Cu") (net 1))
 (segment (start 135.900603 67.649397) (end 135.9 67.65) (width 0.3) (layer "B.Cu") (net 1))
 (segment (start 140.374397 65.65) (end 135.9 65.65) (width 0.3) (layer "B.Cu") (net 1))
 (segment (start 138.175 66.65) (end 133.9 66.65) (width 0.3) (layer "B.Cu") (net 1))
 (segment (start 129.4 65.65) (end 135.9 65.65) (width 0.3) (layer "B.Cu") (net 1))
 (segment (start 140.375 67.649397) (end 135.900603 67.649397) (width 0.3) (layer "B.Cu") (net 1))
 (segment (start 138.175 68.65) (end 133.9 68.65) (width 0.3) (layer "B.Cu") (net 1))
 (segment (start 131.4 68.65) (end 133.9 68.65) (width 0.3) (layer "B.Cu") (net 1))
 (segment (start 140.375 65.649397) (end 140.374397 65.65) (width 0.3) (layer "B.Cu") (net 1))
 (segment (start 129.4 67.65) (end 135.9 67.65) (width 0.3) (layer "B.Cu") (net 1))
 (segment (start 129.4 69.65) (end 135.9 69.65) (width 0.3) (layer "B.Cu") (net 9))
 (segment (start 140.374397 69.65) (end 135.9 69.65) (width 0.3) (layer "B.Cu") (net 9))
 (segment (start 140.375 69.649397) (end 140.374397 69.65) (width 0.3) (layer "B.Cu") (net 9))
 (segment (start 140.374397 95.65) (end 135.9 95.65) (width 0.3) (layer "B.Cu") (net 20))
 (segment (start 129.4 95.65) (end 135.9 95.65) (width 0.3) (layer "B.Cu") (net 20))
 (segment (start 140.375 95.649397) (end 140.374397 95.65) (width 0.3) (layer "B.Cu") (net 20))
 (segment (start 129.4 71.65) (end 135.9 71.65) (width 0.3) (layer "B.Cu") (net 5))
 (segment (start 138.175 70.65) (end 133.9 70.65) (width 0.3) (layer "B.Cu") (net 5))
 (segment (start 131.4 72.65) (end 133.9 72.65) (width 0.3) (layer "B.Cu") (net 5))
 (segment (start 140.375 71.649397) (end 135.900603 71.649397) (width 0.3) (layer "B.Cu") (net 5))
 (segment (start 138.175 72.65) (end 133.9 72.65) (width 0.3) (layer "B.Cu") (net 5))
 (segment (start 135.900603 71.649397) (end 135.9 71.65) (width 0.3) (layer "B.Cu") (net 5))
 (segment (start 131.4 70.65) (end 133.9 70.65) (width 0.3) (layer "B.Cu") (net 5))
 (segment (start 131.4 86.65) (end 133.9 86.65) (width 0.3) (layer "B.Cu") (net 6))
 (segment (start 138.175 86.65) (end 133.9 86.65) (width 0.3) (layer "B.Cu") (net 6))
 (segment (start 138.175 78.65) (end 133.9 78.65) (width 0.3) (layer "B.Cu") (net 22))
 (segment (start 131.4 78.65) (end 133.9 78.65) (width 0.3) (layer "B.Cu") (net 22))
 (segment (start 140.375 91.649397) (end 140.374397 91.65) (width 0.3) (layer "B.Cu") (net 3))
 (segment (start 140.374397 91.65) (end 135.9 91.65) (width 0.3) (layer "B.Cu") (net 3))
 (segment (start 129.4 91.65) (end 135.9 91.65) (width 0.3) (layer "B.Cu") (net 3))
 (segment (start 140.374397 83.65) (end 135.9 83.65) (width 0.3) (layer "B.Cu") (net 18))
 (segment (start 140.375 83.649397) (end 140.374397 83.65) (width 0.3) (layer "B.Cu") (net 18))
 (segment (start 129.4 83.65) (end 135.9 83.65) (width 0.3) (layer "B.Cu") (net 18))
 (segment (start 129.4 85.65) (end 135.9 85.65) (width 0.3) (layer "B.Cu") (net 4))
 (segment (start 140.375 85.649397) (end 140.374397 85.65) (width 0.3) (layer "B.Cu") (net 4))
 (segment (start 140.374397 85.65) (end 135.9 85.65) (width 0.3) (layer "B.Cu") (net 4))
 (segment (start 138.175 90.65) (end 133.9 90.65) (width 0.3) (layer "B.Cu") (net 13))
 (segment (start 131.4 90.65) (end 133.9 90.65) (width 0.3) (layer "B.Cu") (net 13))
 (segment (start 140.374397 81.65) (end 135.9 81.65) (width 0.3) (layer "B.Cu") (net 2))
 (segment (start 129.4 81.65) (end 135.9 81.65) (width 0.3) (layer "B.Cu") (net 2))
 (segment (start 140.375 81.649397) (end 140.374397 81.65) (width 0.3) (layer "B.Cu") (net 2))
 (segment (start 133.9 94.65) (end 138.175 94.65) (width 0.3) (layer "B.Cu") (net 8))
 (segment (start 131.4 94.65) (end 133.9 94.65) (width 0.3) (layer "B.Cu") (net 8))
 (segment (start 140.375 87.649397) (end 140.374397 87.65) (width 0.3) (layer "B.Cu") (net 21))
 (segment (start 129.4 87.65) (end 135.9 87.65) (width 0.3) (layer "B.Cu") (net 21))
 (segment (start 140.374397 87.65) (end 135.9 87.65) (width 0.3) (layer "B.Cu") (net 21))
 (segment (start 140.375 73.649397) (end 140.374397 73.65) (width 0.3) (layer "B.Cu") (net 12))
 (segment (start 129.4 73.65) (end 135.9 73.65) (width 0.3) (layer "B.Cu") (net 12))
 (segment (start 140.374397 73.65) (end 135.9 73.65) (width 0.3) (layer "B.Cu") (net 12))
 (segment (start 138.175 74.65) (end 133.9 74.65) (width 0.3) (layer "B.Cu") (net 24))
 (segment (start 131.4 74.65) (end 133.9 74.65) (width 0.3) (layer "B.Cu") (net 24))
 (segment (start 138.175 82.65) (end 133.9 82.65) (width 0.3) (layer "B.Cu") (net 17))
 (segment (start 131.4 82.65) (end 133.9 82.65) (width 0.3) (layer "B.Cu") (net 17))
 (segment (start 138.175 84.65) (end 133.9 84.65) (width 0.3) (layer "B.Cu") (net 23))
 (segment (start 131.4 84.65) (end 133.9 84.65) (width 0.3) (layer "B.Cu") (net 23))
 (segment (start 131.4 96.65) (end 133.9 96.65) (width 0.3) (layer "B.Cu") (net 15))
 (segment (start 133.9 96.65) (end 138.175 96.65) (width 0.3) (layer "B.Cu") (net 15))
 (segment (start 131.4 92.65) (end 133.9 92.65) (width 0.3) (layer "B.Cu") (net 7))
 (segment (start 138.175 92.65) (end 133.9 92.65) (width 0.3) (layer "B.Cu") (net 7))
 (segment (start 129.4 77.65) (end 129.451 77.701) (width 0.3) (layer "B.Cu") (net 11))
 (segment (start 129.451 77.701) (end 135.849 77.701) (width 0.3) (layer "B.Cu") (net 11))
 (segment (start 135.900603 77.649397) (end 135.9 77.65) (width 0.3) (layer "B.Cu") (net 11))
 (segment (start 140.375 77.649397) (end 135.900603 77.649397) (width 0.3) (layer "B.Cu") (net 11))
 (segment (start 135.849 77.701) (end 135.9 77.65) (width 0.3) (layer "B.Cu") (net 11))
 (segment (start 140.374397 79.65) (end 135.9 79.65) (width 0.3) (layer "B.Cu") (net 19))
 (segment (start 129.4 79.65) (end 135.9 79.65) (width 0.3) (layer "B.Cu") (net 19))
 (segment (start 140.375 79.649397) (end 140.374397 79.65) (width 0.3) (layer "B.Cu") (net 19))
 (segment (start 129.4 89.65) (end 135.9 89.65) (width 0.3) (layer "B.Cu") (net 27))
 (segment (start 140.374397 89.65) (end 135.9 89.65) (width 0.3) (layer "B.Cu") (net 27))
 (segment (start 140.375 89.649397) (end 140.374397 89.65) (width 0.3) (layer "B.Cu") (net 27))
 (segment (start 129.4 97.65) (end 135.9 97.65) (width 0.3) (layer "B.Cu") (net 16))
 (segment (start 140.374397 97.65) (end 135.9 97.65) (width 0.3) (layer "B.Cu") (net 16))
 (segment (start 140.375 97.649397) (end 140.374397 97.65) (width 0.3) (layer "B.Cu") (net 16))
 (segment (start 138.175 64.65) (end 133.9 64.65) (width 0.3) (layer "B.Cu") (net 25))
 (segment (start 131.4 64.65) (end 133.9 64.65) (width 0.3) (layer "B.Cu") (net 25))
 (segment (start 140.374397 93.65) (end 140.375 93.649397) (width 0.3) (layer "B.Cu") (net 10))
 (segment (start 129.4 93.65) (end 135.9 93.65) (width 0.3) (layer "B.Cu") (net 10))
 (segment (start 135.9 93.65) (end 140.374397 93.65) (width 0.3) (layer "B.Cu") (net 10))
 (segment (start 138.175 88.65) (end 133.9 88.65) (width 0.3) (layer "B.Cu") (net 26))
 (segment (start 131.4 88.65) (end 133.9 88.65) (width 0.3) (layer "B.Cu") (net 26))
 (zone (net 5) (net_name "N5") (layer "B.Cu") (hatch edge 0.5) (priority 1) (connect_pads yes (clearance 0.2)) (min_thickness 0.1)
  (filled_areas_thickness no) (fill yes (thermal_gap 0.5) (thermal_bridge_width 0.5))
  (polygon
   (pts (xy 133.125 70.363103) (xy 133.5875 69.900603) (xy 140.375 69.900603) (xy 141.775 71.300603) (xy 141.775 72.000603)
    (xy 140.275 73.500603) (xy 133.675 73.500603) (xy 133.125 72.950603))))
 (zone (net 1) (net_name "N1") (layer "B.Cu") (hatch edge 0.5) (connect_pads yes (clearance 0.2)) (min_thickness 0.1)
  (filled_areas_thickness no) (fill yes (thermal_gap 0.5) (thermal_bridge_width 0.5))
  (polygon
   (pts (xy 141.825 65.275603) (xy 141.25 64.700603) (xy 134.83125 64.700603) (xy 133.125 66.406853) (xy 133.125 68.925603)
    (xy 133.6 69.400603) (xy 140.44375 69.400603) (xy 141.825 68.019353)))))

